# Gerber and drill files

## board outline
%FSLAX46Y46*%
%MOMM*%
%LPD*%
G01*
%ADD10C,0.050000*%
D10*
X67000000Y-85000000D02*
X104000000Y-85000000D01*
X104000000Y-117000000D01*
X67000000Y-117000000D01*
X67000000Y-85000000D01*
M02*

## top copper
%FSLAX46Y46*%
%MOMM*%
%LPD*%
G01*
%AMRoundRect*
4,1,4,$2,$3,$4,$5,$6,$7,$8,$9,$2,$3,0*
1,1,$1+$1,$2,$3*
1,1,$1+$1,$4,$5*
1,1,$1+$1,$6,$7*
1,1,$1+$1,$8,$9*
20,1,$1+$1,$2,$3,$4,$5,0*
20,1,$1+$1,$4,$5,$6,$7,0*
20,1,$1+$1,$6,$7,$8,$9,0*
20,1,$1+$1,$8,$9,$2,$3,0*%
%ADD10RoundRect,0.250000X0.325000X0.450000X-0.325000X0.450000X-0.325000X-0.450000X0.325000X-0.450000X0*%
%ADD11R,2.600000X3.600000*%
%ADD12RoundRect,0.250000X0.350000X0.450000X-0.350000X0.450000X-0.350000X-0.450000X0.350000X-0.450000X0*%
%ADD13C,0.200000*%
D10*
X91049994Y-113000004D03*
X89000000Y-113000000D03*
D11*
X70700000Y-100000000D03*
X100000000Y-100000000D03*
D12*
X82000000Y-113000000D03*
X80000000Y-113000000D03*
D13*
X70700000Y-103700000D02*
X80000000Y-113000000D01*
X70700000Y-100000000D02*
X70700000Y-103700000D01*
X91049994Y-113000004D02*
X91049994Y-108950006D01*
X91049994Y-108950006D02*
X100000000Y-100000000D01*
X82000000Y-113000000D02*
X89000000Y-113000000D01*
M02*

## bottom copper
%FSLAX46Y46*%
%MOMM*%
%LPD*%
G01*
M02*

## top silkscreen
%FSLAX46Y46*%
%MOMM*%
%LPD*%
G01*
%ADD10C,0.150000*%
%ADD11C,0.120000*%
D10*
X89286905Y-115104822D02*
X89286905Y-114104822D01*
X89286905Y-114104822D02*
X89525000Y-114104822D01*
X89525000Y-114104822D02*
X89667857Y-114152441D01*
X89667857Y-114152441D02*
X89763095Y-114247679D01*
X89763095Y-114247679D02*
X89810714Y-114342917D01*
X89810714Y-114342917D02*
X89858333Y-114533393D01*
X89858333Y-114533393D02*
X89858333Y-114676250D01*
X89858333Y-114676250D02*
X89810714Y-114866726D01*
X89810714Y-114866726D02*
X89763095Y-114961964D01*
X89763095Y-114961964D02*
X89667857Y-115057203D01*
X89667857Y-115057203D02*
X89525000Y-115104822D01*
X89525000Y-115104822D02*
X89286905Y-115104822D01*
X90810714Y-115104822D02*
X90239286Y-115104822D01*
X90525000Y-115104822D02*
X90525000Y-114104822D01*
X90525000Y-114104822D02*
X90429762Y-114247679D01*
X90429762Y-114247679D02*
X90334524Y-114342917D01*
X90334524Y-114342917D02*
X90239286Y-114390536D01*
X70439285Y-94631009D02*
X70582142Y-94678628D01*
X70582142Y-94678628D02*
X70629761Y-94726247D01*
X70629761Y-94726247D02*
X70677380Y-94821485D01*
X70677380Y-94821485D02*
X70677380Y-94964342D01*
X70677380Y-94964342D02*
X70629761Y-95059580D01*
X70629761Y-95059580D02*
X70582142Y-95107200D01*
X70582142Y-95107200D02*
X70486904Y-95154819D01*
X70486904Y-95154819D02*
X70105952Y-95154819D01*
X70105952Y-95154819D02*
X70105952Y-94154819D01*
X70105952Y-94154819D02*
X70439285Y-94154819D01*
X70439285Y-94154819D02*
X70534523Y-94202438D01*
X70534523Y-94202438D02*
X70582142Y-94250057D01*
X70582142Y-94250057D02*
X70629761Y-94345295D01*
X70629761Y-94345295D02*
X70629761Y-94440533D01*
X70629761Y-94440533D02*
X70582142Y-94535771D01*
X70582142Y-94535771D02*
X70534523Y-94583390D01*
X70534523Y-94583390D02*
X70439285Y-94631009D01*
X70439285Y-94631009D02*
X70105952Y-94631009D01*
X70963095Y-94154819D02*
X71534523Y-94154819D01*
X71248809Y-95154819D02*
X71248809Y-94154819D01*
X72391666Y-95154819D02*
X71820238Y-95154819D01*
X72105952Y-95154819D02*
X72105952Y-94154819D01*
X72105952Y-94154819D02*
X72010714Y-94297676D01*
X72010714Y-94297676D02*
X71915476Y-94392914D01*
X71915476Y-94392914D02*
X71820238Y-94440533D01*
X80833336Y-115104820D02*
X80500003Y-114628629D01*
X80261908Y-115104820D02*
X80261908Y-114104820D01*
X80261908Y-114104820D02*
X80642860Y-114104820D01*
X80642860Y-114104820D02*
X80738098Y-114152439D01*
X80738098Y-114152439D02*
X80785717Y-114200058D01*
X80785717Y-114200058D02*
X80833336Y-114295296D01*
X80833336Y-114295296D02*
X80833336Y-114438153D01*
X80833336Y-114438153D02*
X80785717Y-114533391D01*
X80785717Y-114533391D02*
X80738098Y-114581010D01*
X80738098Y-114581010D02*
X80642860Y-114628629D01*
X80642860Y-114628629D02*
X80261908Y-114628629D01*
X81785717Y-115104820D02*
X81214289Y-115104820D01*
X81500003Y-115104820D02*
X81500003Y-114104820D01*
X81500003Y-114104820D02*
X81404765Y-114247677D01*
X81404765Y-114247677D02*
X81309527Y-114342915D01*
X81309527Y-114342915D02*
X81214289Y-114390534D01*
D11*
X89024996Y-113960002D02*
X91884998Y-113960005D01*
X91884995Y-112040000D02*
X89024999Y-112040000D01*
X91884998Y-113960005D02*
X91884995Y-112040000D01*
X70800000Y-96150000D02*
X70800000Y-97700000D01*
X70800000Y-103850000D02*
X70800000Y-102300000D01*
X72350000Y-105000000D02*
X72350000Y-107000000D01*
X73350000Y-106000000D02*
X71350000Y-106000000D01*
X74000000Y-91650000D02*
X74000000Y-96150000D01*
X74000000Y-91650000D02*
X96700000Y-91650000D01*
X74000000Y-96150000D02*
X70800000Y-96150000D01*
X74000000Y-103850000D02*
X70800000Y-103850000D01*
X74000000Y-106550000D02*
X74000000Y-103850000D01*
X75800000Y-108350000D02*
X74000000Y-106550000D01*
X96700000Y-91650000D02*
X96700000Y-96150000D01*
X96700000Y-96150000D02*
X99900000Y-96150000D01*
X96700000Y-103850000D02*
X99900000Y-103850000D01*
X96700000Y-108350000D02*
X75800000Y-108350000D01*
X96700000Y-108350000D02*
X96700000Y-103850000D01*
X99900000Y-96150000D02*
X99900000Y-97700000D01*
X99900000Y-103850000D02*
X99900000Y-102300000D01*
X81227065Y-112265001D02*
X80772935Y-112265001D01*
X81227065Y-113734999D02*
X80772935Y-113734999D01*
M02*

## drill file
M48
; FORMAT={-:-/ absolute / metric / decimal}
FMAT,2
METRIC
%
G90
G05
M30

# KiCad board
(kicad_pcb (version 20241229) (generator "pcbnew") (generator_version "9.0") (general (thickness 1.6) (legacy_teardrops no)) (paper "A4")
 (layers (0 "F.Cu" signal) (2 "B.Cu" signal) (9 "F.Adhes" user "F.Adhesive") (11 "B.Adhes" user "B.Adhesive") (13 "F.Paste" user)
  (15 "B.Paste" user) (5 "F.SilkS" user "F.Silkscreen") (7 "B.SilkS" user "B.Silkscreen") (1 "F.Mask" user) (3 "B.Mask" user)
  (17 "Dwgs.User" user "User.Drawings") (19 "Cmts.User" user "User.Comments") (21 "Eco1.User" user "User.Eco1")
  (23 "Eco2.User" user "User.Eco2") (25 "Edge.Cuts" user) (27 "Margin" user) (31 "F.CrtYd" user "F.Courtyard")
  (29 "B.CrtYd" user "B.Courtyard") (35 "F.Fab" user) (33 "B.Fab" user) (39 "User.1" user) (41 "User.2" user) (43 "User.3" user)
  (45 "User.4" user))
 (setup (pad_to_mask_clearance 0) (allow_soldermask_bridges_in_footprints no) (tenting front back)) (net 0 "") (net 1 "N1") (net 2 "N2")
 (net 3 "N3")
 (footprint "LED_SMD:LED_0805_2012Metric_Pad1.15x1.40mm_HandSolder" (layer "F.Cu") (at 90.024997 113.000002 180)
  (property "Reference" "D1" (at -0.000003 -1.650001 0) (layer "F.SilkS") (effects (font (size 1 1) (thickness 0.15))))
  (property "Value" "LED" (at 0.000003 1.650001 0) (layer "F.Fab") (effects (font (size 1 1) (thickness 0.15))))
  (fp_line (start 1.000001 -0.96) (end -1.860001 -0.960003) (stroke (width 0.12) (type solid)) (layer "F.SilkS"))
  (fp_line (start -1.859998 0.960002) (end 0.999998 0.960002) (stroke (width 0.12) (type solid)) (layer "F.SilkS"))
  (fp_line (start -1.860001 -0.960003) (end -1.859998 0.960002) (stroke (width 0.12) (type solid)) (layer "F.SilkS"))
  (pad "1" smd roundrect (at -1.024997 -0.000002 180) (size 1.15 1.4) (layers "F.Cu" "F.Mask" "F.Paste") (roundrect_rratio 0.217391)
   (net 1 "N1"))
  (pad "2" smd roundrect (at 1.024997 0.000002 180) (size 1.15 1.4) (layers "F.Cu" "F.Mask" "F.Paste") (roundrect_rratio 0.217391)
   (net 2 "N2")))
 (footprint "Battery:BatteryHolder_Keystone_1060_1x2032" (layer "F.Cu") (at 85.35 100)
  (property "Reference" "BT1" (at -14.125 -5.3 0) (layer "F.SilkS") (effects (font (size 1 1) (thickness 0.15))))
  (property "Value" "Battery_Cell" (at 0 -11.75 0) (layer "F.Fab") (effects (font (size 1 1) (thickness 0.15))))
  (fp_line (start -14.55 -3.85) (end -14.55 -2.3) (stroke (width 0.12) (type solid)) (layer "F.SilkS"))
  (fp_line (start -14.55 3.85) (end -14.55 2.3) (stroke (width 0.12) (type solid)) (layer "F.SilkS"))
  (fp_line (start -13 5) (end -13 7) (stroke (width 0.12) (type solid)) (layer "F.SilkS"))
  (fp_line (start -12 6) (end -14 6) (stroke (width 0.12) (type solid)) (layer "F.SilkS"))
  (fp_line (start -11.35 -8.35) (end -11.35 -3.85) (stroke (width 0.12) (type solid)) (layer "F.SilkS"))
  (fp_line (start -11.35 -8.35) (end 11.35 -8.35) (stroke (width 0.12) (type solid)) (layer "F.SilkS"))
  (fp_line (start -11.35 -3.85) (end -14.55 -3.85) (stroke (width 0.12) (type solid)) (layer "F.SilkS"))
  (fp_line (start -11.35 3.85) (end -14.55 3.85) (stroke (width 0.12) (type solid)) (layer "F.SilkS"))
  (fp_line (start -11.35 6.55) (end -11.35 3.85) (stroke (width 0.12) (type solid)) (layer "F.SilkS"))
  (fp_line (start -9.55 8.35) (end -11.35 6.55) (stroke (width 0.12) (type solid)) (layer "F.SilkS"))
  (fp_line (start 11.35 -8.35) (end 11.35 -3.85) (stroke (width 0.12) (type solid)) (layer "F.SilkS"))
  (fp_line (start 11.35 -3.85) (end 14.55 -3.85) (stroke (width 0.12) (type solid)) (layer "F.SilkS"))
  (fp_line (start 11.35 3.85) (end 14.55 3.85) (stroke (width 0.12) (type solid)) (layer "F.SilkS"))
  (fp_line (start 11.35 8.35) (end -9.55 8.35) (stroke (width 0.12) (type solid)) (layer "F.SilkS"))
  (fp_line (start 11.35 8.35) (end 11.35 3.85) (stroke (width 0.12) (type solid)) (layer "F.SilkS"))
  (fp_line (start 14.55 -3.85) (end 14.55 -2.3) (stroke (width 0.12) (type solid)) (layer "F.SilkS"))
  (fp_line (start 14.55 3.85) (end 14.55 2.3) (stroke (width 0.12) (type solid)) (layer "F.SilkS"))
  (pad "1" smd rect (at -14.65 0 180) (size 2.6 3.6) (layers "F.Cu" "F.Mask" "F.Paste") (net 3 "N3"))
  (pad "2" smd rect (at 14.65 0 180) (size 2.6 3.6) (layers "F.Cu" "F.Mask" "F.Paste") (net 1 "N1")))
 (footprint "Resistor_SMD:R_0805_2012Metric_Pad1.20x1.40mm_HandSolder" (layer "F.Cu") (at 81 113 180)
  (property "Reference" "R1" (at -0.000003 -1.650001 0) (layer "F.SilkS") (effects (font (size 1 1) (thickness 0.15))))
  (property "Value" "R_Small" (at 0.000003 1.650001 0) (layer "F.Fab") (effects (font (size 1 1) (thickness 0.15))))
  (fp_line (start -0.227065 0.734999) (end 0.227065 0.734999) (stroke (width 0.12) (type solid)) (layer "F.SilkS"))
  (fp_line (start -0.227065 -0.734999) (end 0.227065 -0.734999) (stroke (width 0.12) (type solid)) (layer "F.SilkS"))
  (pad "1" smd roundrect (at -1 0 180) (size 1.2 1.4) (layers "F.Cu" "F.Mask" "F.Paste") (roundrect_rratio 0.208333) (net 2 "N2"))
  (pad "2" smd roundrect (at 1 0 180) (size 1.2 1.4) (layers "F.Cu" "F.Mask" "F.Paste") (roundrect_rratio 0.208333) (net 3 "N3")))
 (gr_rect (start 67 85) (end 104 117) (stroke (width 0.05) (type default)) (fill no) (layer "Edge.Cuts"))
 (segment (start 70.7 103.7) (end 80 113) (width 0.2) (layer "F.Cu") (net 3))
 (segment (start 70.7 100) (end 70.7 103.7) (width 0.2) (layer "F.Cu") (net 3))
 (segment (start 91.049994 113.000004) (end 91.049994 108.950006) (width 0.2) (layer "F.Cu") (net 1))
 (segment (start 91.049994 108.950006) (end 100 100) (width 0.2) (layer "F.Cu") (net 1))
 (segment (start 82 113) (end 89 113) (width 0.2) (layer "F.Cu") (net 2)))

